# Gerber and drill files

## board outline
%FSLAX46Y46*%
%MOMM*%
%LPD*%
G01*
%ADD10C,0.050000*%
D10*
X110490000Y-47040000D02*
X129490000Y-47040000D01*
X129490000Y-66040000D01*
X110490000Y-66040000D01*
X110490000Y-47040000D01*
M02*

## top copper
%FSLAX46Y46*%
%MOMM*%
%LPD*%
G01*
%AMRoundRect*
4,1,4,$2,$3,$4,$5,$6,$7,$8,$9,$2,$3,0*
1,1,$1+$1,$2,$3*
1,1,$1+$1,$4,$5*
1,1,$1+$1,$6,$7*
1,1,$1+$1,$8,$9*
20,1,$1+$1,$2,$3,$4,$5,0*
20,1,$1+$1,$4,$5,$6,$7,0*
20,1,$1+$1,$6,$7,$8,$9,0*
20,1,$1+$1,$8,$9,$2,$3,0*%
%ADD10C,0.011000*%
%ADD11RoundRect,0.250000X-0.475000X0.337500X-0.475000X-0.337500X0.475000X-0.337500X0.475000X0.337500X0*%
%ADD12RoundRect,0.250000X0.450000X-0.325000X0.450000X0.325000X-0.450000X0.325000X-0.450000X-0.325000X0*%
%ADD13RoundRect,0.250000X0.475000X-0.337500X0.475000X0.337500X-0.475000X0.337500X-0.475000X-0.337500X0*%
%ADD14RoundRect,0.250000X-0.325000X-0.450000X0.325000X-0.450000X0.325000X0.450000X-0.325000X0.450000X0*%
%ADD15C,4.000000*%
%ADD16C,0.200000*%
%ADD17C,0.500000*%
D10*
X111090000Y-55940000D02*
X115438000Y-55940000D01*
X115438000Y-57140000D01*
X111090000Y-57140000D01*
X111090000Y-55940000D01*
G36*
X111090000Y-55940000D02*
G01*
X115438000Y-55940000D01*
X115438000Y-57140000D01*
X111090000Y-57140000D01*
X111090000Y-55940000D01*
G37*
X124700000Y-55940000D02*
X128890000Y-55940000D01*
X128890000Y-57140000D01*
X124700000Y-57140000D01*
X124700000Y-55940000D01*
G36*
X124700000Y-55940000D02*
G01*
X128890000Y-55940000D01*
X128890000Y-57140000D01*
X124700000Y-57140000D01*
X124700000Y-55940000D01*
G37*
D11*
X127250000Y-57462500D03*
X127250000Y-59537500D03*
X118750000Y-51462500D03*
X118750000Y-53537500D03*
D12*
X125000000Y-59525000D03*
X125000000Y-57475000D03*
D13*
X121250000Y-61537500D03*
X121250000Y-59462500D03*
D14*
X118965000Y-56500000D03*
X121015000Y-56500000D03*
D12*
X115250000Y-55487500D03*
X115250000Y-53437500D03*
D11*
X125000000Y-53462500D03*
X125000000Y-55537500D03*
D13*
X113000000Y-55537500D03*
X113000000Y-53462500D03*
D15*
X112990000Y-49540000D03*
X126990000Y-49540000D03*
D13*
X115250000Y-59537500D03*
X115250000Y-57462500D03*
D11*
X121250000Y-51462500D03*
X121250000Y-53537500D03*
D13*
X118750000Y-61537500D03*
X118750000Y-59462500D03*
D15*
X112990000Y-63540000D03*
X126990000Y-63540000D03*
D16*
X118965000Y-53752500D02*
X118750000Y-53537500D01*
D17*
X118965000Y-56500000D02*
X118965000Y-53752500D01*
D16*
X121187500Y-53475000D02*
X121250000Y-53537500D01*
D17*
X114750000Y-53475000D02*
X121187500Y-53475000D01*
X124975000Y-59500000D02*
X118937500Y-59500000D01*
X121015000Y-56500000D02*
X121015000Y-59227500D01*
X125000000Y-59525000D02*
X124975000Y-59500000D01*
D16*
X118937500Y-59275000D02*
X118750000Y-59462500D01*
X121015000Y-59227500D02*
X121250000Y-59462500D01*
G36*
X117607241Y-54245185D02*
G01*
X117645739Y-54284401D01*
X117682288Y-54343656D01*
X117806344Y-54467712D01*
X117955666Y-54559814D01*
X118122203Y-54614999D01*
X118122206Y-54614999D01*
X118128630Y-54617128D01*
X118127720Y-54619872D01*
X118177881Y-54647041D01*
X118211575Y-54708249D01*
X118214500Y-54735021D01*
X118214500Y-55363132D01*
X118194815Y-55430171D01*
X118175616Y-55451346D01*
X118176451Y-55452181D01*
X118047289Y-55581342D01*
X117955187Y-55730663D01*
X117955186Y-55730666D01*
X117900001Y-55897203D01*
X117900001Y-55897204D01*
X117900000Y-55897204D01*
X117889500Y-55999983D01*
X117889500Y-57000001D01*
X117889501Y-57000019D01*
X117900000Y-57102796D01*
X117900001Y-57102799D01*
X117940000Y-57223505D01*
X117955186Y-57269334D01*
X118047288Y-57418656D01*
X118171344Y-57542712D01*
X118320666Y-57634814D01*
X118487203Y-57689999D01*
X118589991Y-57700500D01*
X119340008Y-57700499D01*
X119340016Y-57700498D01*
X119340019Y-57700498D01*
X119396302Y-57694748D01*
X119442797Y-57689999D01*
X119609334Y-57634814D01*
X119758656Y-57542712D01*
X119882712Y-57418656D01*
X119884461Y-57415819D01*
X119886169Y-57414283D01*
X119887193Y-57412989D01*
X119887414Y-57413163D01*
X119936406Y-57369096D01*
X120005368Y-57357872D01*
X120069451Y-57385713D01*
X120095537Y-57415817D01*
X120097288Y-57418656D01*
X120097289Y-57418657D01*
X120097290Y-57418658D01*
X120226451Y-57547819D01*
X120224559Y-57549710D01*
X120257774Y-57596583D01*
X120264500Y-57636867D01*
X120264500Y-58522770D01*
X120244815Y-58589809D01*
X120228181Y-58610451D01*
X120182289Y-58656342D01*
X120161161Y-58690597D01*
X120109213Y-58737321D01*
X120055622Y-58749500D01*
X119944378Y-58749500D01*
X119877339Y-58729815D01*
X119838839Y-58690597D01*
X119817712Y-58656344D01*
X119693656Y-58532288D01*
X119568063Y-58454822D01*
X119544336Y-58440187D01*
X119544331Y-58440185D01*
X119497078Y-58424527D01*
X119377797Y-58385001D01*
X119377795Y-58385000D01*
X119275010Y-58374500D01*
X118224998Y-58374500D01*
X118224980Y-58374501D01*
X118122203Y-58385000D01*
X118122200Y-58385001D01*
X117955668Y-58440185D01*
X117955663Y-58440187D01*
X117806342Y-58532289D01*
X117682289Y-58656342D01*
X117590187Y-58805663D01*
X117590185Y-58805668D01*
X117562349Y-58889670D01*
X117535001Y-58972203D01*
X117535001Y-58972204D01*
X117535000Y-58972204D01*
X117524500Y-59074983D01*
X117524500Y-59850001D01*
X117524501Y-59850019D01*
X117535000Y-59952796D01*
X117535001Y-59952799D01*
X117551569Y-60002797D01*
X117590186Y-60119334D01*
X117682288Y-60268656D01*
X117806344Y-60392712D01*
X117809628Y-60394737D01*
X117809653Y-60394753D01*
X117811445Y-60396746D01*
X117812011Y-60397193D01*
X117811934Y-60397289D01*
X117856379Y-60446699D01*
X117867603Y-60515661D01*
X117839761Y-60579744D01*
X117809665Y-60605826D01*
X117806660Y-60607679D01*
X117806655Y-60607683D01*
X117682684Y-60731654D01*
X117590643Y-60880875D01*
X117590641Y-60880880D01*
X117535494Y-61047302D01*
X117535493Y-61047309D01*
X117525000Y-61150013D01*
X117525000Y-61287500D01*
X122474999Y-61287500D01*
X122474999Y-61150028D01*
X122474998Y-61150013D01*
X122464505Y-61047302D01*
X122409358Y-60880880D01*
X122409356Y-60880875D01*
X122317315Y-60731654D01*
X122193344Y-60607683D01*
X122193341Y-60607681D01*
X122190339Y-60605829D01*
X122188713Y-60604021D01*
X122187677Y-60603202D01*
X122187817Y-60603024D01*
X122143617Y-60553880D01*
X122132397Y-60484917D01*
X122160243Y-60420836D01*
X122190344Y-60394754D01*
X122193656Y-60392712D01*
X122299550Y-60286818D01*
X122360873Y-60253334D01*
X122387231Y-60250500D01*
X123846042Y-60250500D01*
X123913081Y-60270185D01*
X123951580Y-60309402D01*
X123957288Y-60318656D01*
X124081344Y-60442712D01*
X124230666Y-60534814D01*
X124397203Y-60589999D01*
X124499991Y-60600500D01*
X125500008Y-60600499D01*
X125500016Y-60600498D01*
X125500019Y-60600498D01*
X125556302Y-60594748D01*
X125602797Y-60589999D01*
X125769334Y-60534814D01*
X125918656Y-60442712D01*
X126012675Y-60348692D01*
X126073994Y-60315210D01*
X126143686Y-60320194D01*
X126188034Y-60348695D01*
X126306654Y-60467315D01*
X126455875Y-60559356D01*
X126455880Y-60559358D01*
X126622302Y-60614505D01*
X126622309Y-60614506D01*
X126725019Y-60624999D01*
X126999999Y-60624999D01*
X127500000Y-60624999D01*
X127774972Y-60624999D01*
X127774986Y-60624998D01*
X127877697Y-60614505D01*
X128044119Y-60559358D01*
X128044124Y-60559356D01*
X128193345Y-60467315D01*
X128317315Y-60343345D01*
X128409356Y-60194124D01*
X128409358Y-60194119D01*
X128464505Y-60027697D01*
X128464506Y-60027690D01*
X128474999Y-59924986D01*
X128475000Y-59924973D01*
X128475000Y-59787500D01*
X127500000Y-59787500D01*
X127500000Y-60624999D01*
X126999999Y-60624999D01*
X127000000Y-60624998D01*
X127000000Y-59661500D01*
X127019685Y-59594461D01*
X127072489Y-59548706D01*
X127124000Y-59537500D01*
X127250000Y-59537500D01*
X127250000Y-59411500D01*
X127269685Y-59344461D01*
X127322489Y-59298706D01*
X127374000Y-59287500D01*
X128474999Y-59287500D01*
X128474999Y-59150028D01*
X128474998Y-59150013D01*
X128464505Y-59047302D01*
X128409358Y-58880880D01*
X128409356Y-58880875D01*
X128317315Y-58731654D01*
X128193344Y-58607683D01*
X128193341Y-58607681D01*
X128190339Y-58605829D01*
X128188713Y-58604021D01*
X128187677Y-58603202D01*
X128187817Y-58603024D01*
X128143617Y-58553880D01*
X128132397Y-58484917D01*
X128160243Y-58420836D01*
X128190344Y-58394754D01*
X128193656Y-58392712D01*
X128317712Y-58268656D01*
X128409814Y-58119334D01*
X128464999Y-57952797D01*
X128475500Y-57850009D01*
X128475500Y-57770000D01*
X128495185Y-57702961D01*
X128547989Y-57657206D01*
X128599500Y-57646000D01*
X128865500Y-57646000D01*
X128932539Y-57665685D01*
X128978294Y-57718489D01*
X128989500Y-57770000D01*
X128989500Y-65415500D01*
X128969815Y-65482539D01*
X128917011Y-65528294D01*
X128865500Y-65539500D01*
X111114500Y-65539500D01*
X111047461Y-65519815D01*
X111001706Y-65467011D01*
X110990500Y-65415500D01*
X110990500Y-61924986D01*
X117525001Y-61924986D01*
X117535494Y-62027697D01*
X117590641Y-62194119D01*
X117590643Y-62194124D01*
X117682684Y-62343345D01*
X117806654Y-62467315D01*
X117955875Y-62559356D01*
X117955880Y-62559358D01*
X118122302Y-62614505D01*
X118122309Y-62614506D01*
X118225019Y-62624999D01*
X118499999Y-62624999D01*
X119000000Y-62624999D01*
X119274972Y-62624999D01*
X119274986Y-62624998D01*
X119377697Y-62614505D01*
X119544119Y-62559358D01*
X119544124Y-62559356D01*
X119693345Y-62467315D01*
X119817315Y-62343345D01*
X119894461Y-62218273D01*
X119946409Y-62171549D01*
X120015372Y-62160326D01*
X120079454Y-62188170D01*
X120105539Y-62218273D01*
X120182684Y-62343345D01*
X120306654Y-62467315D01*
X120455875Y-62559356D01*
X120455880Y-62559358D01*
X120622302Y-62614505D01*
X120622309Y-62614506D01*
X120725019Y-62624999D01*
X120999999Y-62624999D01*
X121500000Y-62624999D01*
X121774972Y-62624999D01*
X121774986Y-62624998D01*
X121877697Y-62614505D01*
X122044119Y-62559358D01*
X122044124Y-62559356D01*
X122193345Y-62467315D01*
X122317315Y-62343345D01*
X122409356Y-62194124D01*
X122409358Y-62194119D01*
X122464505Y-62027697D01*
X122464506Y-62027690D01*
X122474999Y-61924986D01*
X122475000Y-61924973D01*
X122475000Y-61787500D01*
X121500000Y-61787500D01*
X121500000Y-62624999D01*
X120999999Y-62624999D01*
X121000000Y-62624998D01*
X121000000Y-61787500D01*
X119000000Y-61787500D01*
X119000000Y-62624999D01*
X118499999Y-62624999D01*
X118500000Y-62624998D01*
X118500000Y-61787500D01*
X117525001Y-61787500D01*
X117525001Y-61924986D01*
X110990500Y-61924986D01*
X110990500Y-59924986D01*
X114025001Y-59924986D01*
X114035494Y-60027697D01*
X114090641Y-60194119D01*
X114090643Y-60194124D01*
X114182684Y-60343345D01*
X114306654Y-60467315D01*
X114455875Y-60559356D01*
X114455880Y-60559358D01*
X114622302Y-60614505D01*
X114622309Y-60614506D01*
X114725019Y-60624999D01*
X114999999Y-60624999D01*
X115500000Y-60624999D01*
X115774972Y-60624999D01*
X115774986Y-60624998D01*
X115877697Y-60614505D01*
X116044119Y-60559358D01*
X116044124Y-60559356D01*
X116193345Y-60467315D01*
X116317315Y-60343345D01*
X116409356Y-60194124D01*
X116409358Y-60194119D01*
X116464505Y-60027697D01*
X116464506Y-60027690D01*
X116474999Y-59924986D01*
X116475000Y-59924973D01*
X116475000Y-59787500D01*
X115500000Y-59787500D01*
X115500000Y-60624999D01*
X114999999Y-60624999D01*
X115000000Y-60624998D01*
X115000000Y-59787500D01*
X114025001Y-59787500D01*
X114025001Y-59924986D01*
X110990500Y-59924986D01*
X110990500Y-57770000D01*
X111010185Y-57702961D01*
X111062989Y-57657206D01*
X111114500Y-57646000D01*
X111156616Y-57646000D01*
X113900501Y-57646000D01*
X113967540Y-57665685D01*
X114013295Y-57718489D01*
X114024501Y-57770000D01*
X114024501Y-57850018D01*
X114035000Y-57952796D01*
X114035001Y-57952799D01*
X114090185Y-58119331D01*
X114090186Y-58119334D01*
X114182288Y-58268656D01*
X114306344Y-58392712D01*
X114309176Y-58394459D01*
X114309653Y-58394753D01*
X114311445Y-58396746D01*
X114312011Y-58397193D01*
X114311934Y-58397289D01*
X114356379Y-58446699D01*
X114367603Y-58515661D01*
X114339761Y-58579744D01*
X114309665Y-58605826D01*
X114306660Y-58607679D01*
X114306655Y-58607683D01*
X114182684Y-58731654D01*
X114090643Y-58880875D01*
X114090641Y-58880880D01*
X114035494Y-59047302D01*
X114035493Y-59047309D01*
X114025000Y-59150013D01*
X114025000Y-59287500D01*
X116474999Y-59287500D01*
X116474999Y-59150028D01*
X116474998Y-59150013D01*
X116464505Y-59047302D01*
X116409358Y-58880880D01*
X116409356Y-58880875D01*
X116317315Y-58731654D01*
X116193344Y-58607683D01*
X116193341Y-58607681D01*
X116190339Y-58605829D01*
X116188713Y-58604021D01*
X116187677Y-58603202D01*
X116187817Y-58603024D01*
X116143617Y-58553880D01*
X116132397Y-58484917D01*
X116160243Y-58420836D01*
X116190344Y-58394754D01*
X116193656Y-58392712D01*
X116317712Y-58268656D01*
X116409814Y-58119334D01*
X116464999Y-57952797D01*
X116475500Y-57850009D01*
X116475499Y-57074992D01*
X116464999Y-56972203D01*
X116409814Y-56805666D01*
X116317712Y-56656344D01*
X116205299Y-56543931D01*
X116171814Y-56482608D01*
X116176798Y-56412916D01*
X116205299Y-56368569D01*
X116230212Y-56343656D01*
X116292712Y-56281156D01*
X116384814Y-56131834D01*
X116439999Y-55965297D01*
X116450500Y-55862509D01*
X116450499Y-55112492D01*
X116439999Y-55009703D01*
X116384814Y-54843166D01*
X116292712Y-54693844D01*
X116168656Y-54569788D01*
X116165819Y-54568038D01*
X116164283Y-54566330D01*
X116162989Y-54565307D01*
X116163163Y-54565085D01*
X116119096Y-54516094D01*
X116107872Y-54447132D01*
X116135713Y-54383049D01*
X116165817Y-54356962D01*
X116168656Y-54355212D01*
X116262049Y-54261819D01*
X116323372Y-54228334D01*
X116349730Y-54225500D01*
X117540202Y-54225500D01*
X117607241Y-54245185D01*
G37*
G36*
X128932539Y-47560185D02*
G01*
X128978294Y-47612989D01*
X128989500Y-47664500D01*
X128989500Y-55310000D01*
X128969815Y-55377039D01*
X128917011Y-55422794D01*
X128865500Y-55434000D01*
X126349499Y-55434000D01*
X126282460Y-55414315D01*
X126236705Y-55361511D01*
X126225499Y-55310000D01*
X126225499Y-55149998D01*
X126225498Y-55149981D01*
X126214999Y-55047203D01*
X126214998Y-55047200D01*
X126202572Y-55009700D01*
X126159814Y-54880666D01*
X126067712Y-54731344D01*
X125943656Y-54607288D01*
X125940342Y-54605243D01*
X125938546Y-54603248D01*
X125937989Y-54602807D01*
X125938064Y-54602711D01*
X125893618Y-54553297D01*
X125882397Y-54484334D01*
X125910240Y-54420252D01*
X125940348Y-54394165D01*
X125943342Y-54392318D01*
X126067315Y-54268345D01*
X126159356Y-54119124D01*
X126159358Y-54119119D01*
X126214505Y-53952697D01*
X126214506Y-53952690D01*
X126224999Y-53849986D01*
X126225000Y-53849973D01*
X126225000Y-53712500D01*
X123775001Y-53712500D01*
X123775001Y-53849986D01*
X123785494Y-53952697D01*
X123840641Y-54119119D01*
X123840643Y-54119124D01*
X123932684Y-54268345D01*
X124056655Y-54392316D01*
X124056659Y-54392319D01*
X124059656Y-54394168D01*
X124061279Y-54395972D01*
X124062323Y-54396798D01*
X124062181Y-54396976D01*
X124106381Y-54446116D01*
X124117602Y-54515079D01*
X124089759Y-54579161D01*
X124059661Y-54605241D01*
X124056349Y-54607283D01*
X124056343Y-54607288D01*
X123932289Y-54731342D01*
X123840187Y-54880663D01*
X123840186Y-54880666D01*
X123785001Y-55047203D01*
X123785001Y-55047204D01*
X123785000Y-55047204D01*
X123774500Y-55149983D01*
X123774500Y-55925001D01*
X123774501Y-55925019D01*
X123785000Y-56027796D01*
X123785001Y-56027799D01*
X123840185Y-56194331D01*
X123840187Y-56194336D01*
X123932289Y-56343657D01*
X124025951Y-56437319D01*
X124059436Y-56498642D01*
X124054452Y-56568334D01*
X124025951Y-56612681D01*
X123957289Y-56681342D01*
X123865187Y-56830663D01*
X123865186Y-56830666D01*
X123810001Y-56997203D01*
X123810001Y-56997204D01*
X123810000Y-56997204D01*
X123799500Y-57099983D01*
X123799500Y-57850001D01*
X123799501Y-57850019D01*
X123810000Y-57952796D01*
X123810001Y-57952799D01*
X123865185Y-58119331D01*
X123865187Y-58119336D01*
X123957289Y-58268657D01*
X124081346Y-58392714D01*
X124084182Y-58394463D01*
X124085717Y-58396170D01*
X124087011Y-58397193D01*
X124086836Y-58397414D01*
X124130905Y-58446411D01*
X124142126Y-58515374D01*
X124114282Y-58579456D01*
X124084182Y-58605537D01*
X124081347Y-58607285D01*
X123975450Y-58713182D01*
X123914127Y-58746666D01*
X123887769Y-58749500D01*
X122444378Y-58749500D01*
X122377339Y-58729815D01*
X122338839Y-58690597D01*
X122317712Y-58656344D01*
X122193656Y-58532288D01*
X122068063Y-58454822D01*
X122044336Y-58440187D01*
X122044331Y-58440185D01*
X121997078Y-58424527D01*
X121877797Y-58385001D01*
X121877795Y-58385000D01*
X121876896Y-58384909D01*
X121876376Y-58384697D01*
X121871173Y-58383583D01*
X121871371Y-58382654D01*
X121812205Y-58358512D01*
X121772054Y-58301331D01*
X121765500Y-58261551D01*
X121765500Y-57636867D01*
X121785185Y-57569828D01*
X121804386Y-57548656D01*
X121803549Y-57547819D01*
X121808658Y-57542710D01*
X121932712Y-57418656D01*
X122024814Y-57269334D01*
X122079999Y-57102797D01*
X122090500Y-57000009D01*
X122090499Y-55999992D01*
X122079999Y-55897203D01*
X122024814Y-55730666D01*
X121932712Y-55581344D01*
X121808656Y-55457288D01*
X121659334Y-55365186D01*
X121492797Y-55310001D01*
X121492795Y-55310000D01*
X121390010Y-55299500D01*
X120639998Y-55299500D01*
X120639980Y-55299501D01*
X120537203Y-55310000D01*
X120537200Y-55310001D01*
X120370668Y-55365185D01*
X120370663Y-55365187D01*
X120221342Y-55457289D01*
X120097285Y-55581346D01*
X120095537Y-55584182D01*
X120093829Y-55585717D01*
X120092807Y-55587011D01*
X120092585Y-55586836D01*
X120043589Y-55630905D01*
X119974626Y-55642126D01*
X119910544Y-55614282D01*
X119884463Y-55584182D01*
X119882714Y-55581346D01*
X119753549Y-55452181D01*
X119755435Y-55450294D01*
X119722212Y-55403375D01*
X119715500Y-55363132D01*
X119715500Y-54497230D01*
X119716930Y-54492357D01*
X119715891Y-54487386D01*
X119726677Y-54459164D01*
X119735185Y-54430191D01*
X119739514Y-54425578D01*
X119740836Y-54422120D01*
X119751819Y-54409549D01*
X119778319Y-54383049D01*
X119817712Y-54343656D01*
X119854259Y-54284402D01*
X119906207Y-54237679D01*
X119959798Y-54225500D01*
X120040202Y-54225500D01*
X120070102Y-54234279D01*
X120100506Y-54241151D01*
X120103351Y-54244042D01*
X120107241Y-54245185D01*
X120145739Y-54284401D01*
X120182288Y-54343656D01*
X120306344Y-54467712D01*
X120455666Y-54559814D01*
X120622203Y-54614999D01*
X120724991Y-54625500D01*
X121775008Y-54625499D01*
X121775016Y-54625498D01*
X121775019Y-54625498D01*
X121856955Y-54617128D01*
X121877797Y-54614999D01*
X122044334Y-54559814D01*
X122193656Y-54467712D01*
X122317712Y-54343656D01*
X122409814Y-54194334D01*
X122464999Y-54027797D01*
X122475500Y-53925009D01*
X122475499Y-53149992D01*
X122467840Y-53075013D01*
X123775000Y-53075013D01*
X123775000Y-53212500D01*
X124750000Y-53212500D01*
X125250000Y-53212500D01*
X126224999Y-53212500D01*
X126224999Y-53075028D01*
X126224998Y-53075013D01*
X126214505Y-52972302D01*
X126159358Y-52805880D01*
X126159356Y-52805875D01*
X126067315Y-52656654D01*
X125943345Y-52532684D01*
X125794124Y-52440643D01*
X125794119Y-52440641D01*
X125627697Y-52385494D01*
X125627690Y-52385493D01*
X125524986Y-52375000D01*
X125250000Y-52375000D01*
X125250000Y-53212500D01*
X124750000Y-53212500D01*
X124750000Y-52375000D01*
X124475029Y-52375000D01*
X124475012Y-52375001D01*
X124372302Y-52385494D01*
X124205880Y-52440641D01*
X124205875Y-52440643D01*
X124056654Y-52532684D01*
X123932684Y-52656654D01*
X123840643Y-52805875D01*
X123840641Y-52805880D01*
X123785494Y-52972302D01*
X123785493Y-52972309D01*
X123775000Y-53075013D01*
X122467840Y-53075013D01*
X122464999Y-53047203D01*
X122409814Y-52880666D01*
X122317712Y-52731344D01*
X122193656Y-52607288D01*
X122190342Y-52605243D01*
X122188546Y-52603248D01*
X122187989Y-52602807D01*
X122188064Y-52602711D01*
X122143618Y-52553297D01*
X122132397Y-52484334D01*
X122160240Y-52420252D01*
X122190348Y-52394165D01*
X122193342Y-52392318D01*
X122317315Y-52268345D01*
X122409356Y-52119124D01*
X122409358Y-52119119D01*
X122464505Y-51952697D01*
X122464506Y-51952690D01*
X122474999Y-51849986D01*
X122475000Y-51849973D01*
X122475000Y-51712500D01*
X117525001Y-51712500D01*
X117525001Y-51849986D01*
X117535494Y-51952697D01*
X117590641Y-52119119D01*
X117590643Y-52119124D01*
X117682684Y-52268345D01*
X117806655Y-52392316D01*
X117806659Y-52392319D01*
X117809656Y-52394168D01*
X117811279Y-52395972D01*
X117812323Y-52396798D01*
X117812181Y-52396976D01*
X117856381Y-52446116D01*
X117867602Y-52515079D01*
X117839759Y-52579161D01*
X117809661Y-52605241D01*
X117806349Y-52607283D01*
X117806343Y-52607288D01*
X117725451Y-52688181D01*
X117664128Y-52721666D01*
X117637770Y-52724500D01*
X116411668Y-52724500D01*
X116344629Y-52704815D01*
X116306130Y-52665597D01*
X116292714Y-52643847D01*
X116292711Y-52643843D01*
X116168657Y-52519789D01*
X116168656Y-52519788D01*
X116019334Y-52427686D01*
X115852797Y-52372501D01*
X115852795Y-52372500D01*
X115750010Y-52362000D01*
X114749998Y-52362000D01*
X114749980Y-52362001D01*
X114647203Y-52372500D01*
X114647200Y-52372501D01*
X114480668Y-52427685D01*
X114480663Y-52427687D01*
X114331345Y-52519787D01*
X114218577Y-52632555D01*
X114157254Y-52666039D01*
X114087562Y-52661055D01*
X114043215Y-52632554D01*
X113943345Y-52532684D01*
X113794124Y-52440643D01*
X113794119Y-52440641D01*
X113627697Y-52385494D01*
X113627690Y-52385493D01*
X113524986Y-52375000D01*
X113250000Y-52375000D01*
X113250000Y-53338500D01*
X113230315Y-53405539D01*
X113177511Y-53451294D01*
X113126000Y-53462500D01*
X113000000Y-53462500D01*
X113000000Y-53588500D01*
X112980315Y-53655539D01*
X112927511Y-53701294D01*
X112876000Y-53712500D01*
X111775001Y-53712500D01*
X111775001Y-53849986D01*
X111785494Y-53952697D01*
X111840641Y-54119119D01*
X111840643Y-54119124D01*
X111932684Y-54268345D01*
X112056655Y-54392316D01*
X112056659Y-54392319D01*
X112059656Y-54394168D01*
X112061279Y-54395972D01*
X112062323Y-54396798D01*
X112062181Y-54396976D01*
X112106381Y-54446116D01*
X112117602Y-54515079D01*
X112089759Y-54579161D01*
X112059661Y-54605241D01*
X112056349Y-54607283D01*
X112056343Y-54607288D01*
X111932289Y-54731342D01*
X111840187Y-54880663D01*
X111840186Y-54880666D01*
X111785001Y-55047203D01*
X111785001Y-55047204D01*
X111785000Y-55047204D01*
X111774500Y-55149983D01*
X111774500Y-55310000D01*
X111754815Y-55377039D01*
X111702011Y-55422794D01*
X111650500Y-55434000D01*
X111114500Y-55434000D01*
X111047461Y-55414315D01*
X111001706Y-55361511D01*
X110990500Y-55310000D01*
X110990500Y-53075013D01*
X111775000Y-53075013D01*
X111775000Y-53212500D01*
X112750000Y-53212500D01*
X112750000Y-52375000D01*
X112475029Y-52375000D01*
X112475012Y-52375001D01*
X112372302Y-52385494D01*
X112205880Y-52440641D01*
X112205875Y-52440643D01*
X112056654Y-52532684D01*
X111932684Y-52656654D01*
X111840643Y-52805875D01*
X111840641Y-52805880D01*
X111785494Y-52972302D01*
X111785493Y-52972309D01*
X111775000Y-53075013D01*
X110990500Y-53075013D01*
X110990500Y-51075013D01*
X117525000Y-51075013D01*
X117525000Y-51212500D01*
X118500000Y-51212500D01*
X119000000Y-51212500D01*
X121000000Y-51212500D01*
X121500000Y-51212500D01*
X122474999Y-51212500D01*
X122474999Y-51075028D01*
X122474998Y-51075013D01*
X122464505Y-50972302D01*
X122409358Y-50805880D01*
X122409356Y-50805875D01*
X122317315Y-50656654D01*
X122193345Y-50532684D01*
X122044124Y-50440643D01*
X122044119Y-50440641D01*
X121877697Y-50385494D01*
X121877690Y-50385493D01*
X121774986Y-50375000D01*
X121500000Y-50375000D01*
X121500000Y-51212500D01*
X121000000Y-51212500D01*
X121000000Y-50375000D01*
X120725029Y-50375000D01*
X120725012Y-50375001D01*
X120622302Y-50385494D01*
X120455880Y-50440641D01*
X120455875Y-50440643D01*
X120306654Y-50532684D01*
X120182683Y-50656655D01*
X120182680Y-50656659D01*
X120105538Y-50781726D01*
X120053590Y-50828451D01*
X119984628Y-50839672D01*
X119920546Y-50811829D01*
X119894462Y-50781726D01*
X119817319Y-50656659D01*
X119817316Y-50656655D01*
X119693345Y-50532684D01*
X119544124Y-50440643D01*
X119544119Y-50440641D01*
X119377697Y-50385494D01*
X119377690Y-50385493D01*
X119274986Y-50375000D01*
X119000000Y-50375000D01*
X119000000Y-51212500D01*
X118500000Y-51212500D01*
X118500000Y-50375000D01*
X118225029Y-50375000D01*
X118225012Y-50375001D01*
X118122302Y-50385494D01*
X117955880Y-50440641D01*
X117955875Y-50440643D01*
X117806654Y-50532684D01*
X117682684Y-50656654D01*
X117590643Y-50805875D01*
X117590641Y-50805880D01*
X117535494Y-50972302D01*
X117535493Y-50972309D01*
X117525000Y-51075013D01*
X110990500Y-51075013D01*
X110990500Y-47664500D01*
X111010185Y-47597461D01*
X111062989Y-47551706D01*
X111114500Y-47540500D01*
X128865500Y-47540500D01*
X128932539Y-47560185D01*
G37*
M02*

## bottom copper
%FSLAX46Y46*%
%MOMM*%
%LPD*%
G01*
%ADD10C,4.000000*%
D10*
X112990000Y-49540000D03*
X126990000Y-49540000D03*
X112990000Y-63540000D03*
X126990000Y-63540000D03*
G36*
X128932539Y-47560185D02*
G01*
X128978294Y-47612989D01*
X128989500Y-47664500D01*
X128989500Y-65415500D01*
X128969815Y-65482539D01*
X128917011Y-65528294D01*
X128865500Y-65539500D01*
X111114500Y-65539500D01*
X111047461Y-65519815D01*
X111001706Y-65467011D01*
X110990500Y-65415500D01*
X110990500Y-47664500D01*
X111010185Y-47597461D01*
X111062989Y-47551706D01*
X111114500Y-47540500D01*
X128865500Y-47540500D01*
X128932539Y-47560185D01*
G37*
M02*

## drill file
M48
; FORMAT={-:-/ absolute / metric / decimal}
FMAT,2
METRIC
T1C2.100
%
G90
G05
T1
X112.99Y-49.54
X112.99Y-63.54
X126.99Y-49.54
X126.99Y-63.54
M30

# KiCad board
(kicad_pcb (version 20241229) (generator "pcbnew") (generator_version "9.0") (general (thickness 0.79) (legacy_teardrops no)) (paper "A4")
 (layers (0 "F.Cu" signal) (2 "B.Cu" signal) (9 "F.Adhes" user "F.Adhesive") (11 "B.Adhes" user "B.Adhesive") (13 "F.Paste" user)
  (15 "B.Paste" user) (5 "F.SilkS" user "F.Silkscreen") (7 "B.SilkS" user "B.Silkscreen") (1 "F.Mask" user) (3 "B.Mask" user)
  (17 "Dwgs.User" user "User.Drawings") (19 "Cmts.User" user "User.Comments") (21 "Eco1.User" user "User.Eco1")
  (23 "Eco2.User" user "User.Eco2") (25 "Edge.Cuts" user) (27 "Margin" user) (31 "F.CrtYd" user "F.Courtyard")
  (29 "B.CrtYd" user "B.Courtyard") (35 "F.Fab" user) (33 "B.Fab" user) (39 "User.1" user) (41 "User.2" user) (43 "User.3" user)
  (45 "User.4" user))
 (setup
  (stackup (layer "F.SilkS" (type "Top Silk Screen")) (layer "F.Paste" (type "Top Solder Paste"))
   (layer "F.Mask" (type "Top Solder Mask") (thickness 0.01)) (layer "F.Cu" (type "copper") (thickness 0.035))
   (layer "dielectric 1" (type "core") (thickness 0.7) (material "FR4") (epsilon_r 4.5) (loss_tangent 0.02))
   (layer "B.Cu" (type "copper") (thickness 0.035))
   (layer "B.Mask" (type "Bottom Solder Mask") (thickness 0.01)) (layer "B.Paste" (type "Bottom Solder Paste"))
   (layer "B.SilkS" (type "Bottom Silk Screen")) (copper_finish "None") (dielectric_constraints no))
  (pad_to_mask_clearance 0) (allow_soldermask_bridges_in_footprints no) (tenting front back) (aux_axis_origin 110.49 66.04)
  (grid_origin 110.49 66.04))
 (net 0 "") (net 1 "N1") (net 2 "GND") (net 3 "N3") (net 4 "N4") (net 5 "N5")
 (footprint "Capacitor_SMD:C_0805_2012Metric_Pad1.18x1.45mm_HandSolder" (layer "F.Cu") (at 127.25 58.5 -90)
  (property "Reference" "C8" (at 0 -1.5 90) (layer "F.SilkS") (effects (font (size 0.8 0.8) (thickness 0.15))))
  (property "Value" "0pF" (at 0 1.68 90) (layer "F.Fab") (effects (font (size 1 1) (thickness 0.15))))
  (pad "1" smd roundrect (at -1.0375 0 270) (size 1.175 1.45) (layers "F.Cu" "F.Mask" "F.Paste") (roundrect_rratio 0.212766) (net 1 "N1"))
  (pad "2" smd roundrect (at 1.0375 0 270) (size 1.175 1.45) (layers "F.Cu" "F.Mask" "F.Paste") (roundrect_rratio 0.212766) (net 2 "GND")))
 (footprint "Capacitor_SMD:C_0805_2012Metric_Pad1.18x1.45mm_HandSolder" (layer "F.Cu") (at 118.75 52.5 -90)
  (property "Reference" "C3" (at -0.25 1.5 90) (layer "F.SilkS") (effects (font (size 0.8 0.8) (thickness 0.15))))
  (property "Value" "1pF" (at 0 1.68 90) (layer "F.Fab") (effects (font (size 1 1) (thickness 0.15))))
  (pad "1" smd roundrect (at -1.0375 0 270) (size 1.175 1.45) (layers "F.Cu" "F.Mask" "F.Paste") (roundrect_rratio 0.212766) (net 2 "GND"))
  (pad "2" smd roundrect (at 1.0375 0 270) (size 1.175 1.45) (layers "F.Cu" "F.Mask" "F.Paste") (roundrect_rratio 0.212766) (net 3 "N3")))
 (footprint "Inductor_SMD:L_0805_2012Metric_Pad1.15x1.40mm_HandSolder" (layer "F.Cu") (at 125 58.5 90)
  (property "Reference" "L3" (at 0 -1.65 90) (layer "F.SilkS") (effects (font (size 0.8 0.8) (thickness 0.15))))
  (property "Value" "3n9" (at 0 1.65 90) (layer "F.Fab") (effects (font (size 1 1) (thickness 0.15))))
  (pad "1" smd roundrect (at -1.025 0 90) (size 1.15 1.4) (layers "F.Cu" "F.Mask" "F.Paste") (roundrect_rratio 0.217391) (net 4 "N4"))
  (pad "2" smd roundrect (at 1.025 0 90) (size 1.15 1.4) (layers "F.Cu" "F.Mask" "F.Paste") (roundrect_rratio 0.217391) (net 1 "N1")))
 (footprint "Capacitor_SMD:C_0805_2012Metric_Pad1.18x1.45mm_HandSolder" (layer "F.Cu") (at 121.25 60.5 90)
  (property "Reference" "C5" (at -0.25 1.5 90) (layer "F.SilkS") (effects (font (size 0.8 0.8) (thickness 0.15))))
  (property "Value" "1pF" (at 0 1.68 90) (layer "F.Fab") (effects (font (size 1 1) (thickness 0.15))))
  (pad "1" smd roundrect (at -1.0375 0 90) (size 1.175 1.45) (layers "F.Cu" "F.Mask" "F.Paste") (roundrect_rratio 0.212766) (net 2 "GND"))
  (pad "2" smd roundrect (at 1.0375 0 90) (size 1.175 1.45) (layers "F.Cu" "F.Mask" "F.Paste") (roundrect_rratio 0.212766) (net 4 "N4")))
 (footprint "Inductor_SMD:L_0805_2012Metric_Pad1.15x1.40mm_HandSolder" (layer "F.Cu") (at 119.99 56.5)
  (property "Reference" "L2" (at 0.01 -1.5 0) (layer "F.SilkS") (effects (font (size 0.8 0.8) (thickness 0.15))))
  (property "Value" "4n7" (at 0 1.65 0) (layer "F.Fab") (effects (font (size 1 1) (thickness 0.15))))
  (pad "1" smd roundrect (at -1.025 0) (size 1.15 1.4) (layers "F.Cu" "F.Mask" "F.Paste") (roundrect_rratio 0.217391) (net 3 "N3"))
  (pad "2" smd roundrect (at 1.025 0) (size 1.15 1.4) (layers "F.Cu" "F.Mask" "F.Paste") (roundrect_rratio 0.217391) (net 4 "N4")))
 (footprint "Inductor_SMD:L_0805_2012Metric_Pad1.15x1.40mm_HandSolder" (layer "F.Cu") (at 115.25 54.4625 90)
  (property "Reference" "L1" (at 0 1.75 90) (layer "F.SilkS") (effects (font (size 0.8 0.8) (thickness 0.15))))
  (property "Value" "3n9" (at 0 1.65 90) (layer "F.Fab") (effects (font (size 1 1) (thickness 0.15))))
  (pad "1" smd roundrect (at -1.025 0 90) (size 1.15 1.4) (layers "F.Cu" "F.Mask" "F.Paste") (roundrect_rratio 0.217391) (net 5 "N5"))
  (pad "2" smd roundrect (at 1.025 0 90) (size 1.15 1.4) (layers "F.Cu" "F.Mask" "F.Paste") (roundrect_rratio 0.217391) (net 3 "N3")))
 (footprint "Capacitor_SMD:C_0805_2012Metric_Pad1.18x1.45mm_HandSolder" (layer "F.Cu") (at 125 54.5 -90)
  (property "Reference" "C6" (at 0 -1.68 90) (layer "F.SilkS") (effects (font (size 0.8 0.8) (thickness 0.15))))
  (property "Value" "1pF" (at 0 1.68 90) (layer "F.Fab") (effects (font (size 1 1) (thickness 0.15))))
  (pad "1" smd roundrect (at -1.0375 0 270) (size 1.175 1.45) (layers "F.Cu" "F.Mask" "F.Paste") (roundrect_rratio 0.212766) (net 2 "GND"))
  (pad "2" smd roundrect (at 1.0375 0 270) (size 1.175 1.45) (layers "F.Cu" "F.Mask" "F.Paste") (roundrect_rratio 0.212766) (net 1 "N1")))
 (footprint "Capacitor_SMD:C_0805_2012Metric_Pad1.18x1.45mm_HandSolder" (layer "F.Cu") (at 113 54.5 90)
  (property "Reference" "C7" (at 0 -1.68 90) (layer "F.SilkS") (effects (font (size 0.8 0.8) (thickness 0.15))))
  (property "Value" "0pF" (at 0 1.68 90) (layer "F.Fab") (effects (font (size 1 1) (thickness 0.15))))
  (pad "1" smd roundrect (at -1.0375 0 90) (size 1.175 1.45) (layers "F.Cu" "F.Mask" "F.Paste") (roundrect_rratio 0.212766) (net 5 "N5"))
  (pad "2" smd roundrect (at 1.0375 0 90) (size 1.175 1.45) (layers "F.Cu" "F.Mask" "F.Paste") (roundrect_rratio 0.212766) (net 2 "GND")))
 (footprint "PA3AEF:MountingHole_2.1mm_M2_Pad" (layer "F.Cu") (at 112.99 49.54)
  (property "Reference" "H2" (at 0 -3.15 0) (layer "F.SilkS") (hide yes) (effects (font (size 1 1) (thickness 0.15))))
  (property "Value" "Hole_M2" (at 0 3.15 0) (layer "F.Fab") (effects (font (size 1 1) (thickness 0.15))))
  (pad "1" thru_hole circle (at 0 0) (size 4 4) (drill 2.1) (layers "*.Cu" "*.Mask") (remove_unused_layers no) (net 2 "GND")
   (zone_connect 2)))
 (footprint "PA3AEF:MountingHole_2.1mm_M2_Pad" (layer "F.Cu") (at 126.99 49.54)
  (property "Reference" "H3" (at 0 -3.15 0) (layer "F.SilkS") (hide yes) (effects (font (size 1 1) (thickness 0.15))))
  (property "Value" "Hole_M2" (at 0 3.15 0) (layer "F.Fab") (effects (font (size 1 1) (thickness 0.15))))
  (pad "1" thru_hole circle (at 0 0) (size 4 4) (drill 2.1) (layers "*.Cu" "*.Mask") (remove_unused_layers no) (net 2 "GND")
   (zone_connect 2)))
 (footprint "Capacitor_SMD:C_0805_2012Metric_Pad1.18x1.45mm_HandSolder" (layer "F.Cu") (at 115.25 58.5 90)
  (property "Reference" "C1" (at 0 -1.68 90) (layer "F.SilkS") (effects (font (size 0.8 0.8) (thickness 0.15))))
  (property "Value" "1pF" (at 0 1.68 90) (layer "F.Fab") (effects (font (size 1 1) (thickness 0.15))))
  (pad "1" smd roundrect (at -1.0375 0 90) (size 1.175 1.45) (layers "F.Cu" "F.Mask" "F.Paste") (roundrect_rratio 0.212766) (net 2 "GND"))
  (pad "2" smd roundrect (at 1.0375 0 90) (size 1.175 1.45) (layers "F.Cu" "F.Mask" "F.Paste") (roundrect_rratio 0.212766) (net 5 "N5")))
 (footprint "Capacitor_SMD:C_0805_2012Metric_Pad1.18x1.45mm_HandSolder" (layer "F.Cu") (at 121.25 52.5 -90)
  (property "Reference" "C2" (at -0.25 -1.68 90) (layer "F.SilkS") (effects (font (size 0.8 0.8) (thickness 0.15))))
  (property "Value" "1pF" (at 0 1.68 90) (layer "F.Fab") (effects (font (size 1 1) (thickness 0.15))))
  (pad "1" smd roundrect (at -1.0375 0 270) (size 1.175 1.45) (layers "F.Cu" "F.Mask" "F.Paste") (roundrect_rratio 0.212766) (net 2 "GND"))
  (pad "2" smd roundrect (at 1.0375 0 270) (size 1.175 1.45) (layers "F.Cu" "F.Mask" "F.Paste") (roundrect_rratio 0.212766) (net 3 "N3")))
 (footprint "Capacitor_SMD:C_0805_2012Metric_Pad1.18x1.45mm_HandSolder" (layer "F.Cu") (at 118.75 60.5 90)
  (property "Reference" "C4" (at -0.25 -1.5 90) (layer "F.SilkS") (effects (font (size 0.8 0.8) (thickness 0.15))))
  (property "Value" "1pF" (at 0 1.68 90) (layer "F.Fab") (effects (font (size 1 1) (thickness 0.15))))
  (pad "1" smd roundrect (at -1.0375 0 90) (size 1.175 1.45) (layers "F.Cu" "F.Mask" "F.Paste") (roundrect_rratio 0.212766) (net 2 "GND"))
  (pad "2" smd roundrect (at 1.0375 0 90) (size 1.175 1.45) (layers "F.Cu" "F.Mask" "F.Paste") (roundrect_rratio 0.212766) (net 4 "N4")))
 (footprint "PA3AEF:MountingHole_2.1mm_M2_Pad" (layer "F.Cu") (at 112.99 63.54)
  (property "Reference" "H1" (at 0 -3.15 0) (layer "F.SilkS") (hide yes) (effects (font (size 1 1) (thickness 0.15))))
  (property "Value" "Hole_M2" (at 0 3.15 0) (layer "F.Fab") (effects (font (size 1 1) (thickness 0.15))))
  (pad "1" thru_hole circle (at 0 0) (size 4 4) (drill 2.1) (layers "*.Cu" "*.Mask") (remove_unused_layers no) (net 2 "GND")
   (zone_connect 2)))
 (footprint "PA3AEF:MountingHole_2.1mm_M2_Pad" (layer "F.Cu") (at 126.99 63.54)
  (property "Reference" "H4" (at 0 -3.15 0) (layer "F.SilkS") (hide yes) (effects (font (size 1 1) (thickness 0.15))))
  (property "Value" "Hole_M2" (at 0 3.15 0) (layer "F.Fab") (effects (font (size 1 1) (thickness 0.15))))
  (pad "1" thru_hole circle (at 0 0) (size 4 4) (drill 2.1) (layers "*.Cu" "*.Mask") (remove_unused_layers no) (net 2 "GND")
   (zone_connect 2)))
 (gr_rect (start 111.09 55.94) (end 115.438 57.14) (stroke (width 0.011) (type solid)) (fill yes) (layer "F.Cu") (net 5))
 (gr_rect (start 124.7 55.94) (end 128.89 57.14) (stroke (width 0.011) (type solid)) (fill yes) (layer "F.Cu") (net 1))
 (gr_rect (start 110.49 47.04) (end 129.49 66.04) (stroke (width 0.05) (type solid)) (fill no) (layer "Edge.Cuts"))
 (segment (start 118.965 53.7525) (end 118.75 53.5375) (width 0.2) (layer "F.Cu") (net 3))
 (segment (start 118.965 56.5) (end 118.965 53.7525) (width 0.5) (layer "F.Cu") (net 3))
 (segment (start 121.1875 53.475) (end 121.25 53.5375) (width 0.2) (layer "F.Cu") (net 3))
 (segment (start 114.75 53.475) (end 121.1875 53.475) (width 0.5) (layer "F.Cu") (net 3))
 (segment (start 124.975 59.5) (end 118.9375 59.5) (width 0.5) (layer "F.Cu") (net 4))
 (segment (start 121.015 56.5) (end 121.015 59.2275) (width 0.5) (layer "F.Cu") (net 4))
 (segment (start 125 59.525) (end 124.975 59.5) (width 0.5) (layer "F.Cu") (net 4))
 (segment (start 118.9375 59.275) (end 118.75 59.4625) (width 0.2) (layer "F.Cu") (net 4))
 (segment (start 121.015 59.2275) (end 121.25 59.4625) (width 0.2) (layer "F.Cu") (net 4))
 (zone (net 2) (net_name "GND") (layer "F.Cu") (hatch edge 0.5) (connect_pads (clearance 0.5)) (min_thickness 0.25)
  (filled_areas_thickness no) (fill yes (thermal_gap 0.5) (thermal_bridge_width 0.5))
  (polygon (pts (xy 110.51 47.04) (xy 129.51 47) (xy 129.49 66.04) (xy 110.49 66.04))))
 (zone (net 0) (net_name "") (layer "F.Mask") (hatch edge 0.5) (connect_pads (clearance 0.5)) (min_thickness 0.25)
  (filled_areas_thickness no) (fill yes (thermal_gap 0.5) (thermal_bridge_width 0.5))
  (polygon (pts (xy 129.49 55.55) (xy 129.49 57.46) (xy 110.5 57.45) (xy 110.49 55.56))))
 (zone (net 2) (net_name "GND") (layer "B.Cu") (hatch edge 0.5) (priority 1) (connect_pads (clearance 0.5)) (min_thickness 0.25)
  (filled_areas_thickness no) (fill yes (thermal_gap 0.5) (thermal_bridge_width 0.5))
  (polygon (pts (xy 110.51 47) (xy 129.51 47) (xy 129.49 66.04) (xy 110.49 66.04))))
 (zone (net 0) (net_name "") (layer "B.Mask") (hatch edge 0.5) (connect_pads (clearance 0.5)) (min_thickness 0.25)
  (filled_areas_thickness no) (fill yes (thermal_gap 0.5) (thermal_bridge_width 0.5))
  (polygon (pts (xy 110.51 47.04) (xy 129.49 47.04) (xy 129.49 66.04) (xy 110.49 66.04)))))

